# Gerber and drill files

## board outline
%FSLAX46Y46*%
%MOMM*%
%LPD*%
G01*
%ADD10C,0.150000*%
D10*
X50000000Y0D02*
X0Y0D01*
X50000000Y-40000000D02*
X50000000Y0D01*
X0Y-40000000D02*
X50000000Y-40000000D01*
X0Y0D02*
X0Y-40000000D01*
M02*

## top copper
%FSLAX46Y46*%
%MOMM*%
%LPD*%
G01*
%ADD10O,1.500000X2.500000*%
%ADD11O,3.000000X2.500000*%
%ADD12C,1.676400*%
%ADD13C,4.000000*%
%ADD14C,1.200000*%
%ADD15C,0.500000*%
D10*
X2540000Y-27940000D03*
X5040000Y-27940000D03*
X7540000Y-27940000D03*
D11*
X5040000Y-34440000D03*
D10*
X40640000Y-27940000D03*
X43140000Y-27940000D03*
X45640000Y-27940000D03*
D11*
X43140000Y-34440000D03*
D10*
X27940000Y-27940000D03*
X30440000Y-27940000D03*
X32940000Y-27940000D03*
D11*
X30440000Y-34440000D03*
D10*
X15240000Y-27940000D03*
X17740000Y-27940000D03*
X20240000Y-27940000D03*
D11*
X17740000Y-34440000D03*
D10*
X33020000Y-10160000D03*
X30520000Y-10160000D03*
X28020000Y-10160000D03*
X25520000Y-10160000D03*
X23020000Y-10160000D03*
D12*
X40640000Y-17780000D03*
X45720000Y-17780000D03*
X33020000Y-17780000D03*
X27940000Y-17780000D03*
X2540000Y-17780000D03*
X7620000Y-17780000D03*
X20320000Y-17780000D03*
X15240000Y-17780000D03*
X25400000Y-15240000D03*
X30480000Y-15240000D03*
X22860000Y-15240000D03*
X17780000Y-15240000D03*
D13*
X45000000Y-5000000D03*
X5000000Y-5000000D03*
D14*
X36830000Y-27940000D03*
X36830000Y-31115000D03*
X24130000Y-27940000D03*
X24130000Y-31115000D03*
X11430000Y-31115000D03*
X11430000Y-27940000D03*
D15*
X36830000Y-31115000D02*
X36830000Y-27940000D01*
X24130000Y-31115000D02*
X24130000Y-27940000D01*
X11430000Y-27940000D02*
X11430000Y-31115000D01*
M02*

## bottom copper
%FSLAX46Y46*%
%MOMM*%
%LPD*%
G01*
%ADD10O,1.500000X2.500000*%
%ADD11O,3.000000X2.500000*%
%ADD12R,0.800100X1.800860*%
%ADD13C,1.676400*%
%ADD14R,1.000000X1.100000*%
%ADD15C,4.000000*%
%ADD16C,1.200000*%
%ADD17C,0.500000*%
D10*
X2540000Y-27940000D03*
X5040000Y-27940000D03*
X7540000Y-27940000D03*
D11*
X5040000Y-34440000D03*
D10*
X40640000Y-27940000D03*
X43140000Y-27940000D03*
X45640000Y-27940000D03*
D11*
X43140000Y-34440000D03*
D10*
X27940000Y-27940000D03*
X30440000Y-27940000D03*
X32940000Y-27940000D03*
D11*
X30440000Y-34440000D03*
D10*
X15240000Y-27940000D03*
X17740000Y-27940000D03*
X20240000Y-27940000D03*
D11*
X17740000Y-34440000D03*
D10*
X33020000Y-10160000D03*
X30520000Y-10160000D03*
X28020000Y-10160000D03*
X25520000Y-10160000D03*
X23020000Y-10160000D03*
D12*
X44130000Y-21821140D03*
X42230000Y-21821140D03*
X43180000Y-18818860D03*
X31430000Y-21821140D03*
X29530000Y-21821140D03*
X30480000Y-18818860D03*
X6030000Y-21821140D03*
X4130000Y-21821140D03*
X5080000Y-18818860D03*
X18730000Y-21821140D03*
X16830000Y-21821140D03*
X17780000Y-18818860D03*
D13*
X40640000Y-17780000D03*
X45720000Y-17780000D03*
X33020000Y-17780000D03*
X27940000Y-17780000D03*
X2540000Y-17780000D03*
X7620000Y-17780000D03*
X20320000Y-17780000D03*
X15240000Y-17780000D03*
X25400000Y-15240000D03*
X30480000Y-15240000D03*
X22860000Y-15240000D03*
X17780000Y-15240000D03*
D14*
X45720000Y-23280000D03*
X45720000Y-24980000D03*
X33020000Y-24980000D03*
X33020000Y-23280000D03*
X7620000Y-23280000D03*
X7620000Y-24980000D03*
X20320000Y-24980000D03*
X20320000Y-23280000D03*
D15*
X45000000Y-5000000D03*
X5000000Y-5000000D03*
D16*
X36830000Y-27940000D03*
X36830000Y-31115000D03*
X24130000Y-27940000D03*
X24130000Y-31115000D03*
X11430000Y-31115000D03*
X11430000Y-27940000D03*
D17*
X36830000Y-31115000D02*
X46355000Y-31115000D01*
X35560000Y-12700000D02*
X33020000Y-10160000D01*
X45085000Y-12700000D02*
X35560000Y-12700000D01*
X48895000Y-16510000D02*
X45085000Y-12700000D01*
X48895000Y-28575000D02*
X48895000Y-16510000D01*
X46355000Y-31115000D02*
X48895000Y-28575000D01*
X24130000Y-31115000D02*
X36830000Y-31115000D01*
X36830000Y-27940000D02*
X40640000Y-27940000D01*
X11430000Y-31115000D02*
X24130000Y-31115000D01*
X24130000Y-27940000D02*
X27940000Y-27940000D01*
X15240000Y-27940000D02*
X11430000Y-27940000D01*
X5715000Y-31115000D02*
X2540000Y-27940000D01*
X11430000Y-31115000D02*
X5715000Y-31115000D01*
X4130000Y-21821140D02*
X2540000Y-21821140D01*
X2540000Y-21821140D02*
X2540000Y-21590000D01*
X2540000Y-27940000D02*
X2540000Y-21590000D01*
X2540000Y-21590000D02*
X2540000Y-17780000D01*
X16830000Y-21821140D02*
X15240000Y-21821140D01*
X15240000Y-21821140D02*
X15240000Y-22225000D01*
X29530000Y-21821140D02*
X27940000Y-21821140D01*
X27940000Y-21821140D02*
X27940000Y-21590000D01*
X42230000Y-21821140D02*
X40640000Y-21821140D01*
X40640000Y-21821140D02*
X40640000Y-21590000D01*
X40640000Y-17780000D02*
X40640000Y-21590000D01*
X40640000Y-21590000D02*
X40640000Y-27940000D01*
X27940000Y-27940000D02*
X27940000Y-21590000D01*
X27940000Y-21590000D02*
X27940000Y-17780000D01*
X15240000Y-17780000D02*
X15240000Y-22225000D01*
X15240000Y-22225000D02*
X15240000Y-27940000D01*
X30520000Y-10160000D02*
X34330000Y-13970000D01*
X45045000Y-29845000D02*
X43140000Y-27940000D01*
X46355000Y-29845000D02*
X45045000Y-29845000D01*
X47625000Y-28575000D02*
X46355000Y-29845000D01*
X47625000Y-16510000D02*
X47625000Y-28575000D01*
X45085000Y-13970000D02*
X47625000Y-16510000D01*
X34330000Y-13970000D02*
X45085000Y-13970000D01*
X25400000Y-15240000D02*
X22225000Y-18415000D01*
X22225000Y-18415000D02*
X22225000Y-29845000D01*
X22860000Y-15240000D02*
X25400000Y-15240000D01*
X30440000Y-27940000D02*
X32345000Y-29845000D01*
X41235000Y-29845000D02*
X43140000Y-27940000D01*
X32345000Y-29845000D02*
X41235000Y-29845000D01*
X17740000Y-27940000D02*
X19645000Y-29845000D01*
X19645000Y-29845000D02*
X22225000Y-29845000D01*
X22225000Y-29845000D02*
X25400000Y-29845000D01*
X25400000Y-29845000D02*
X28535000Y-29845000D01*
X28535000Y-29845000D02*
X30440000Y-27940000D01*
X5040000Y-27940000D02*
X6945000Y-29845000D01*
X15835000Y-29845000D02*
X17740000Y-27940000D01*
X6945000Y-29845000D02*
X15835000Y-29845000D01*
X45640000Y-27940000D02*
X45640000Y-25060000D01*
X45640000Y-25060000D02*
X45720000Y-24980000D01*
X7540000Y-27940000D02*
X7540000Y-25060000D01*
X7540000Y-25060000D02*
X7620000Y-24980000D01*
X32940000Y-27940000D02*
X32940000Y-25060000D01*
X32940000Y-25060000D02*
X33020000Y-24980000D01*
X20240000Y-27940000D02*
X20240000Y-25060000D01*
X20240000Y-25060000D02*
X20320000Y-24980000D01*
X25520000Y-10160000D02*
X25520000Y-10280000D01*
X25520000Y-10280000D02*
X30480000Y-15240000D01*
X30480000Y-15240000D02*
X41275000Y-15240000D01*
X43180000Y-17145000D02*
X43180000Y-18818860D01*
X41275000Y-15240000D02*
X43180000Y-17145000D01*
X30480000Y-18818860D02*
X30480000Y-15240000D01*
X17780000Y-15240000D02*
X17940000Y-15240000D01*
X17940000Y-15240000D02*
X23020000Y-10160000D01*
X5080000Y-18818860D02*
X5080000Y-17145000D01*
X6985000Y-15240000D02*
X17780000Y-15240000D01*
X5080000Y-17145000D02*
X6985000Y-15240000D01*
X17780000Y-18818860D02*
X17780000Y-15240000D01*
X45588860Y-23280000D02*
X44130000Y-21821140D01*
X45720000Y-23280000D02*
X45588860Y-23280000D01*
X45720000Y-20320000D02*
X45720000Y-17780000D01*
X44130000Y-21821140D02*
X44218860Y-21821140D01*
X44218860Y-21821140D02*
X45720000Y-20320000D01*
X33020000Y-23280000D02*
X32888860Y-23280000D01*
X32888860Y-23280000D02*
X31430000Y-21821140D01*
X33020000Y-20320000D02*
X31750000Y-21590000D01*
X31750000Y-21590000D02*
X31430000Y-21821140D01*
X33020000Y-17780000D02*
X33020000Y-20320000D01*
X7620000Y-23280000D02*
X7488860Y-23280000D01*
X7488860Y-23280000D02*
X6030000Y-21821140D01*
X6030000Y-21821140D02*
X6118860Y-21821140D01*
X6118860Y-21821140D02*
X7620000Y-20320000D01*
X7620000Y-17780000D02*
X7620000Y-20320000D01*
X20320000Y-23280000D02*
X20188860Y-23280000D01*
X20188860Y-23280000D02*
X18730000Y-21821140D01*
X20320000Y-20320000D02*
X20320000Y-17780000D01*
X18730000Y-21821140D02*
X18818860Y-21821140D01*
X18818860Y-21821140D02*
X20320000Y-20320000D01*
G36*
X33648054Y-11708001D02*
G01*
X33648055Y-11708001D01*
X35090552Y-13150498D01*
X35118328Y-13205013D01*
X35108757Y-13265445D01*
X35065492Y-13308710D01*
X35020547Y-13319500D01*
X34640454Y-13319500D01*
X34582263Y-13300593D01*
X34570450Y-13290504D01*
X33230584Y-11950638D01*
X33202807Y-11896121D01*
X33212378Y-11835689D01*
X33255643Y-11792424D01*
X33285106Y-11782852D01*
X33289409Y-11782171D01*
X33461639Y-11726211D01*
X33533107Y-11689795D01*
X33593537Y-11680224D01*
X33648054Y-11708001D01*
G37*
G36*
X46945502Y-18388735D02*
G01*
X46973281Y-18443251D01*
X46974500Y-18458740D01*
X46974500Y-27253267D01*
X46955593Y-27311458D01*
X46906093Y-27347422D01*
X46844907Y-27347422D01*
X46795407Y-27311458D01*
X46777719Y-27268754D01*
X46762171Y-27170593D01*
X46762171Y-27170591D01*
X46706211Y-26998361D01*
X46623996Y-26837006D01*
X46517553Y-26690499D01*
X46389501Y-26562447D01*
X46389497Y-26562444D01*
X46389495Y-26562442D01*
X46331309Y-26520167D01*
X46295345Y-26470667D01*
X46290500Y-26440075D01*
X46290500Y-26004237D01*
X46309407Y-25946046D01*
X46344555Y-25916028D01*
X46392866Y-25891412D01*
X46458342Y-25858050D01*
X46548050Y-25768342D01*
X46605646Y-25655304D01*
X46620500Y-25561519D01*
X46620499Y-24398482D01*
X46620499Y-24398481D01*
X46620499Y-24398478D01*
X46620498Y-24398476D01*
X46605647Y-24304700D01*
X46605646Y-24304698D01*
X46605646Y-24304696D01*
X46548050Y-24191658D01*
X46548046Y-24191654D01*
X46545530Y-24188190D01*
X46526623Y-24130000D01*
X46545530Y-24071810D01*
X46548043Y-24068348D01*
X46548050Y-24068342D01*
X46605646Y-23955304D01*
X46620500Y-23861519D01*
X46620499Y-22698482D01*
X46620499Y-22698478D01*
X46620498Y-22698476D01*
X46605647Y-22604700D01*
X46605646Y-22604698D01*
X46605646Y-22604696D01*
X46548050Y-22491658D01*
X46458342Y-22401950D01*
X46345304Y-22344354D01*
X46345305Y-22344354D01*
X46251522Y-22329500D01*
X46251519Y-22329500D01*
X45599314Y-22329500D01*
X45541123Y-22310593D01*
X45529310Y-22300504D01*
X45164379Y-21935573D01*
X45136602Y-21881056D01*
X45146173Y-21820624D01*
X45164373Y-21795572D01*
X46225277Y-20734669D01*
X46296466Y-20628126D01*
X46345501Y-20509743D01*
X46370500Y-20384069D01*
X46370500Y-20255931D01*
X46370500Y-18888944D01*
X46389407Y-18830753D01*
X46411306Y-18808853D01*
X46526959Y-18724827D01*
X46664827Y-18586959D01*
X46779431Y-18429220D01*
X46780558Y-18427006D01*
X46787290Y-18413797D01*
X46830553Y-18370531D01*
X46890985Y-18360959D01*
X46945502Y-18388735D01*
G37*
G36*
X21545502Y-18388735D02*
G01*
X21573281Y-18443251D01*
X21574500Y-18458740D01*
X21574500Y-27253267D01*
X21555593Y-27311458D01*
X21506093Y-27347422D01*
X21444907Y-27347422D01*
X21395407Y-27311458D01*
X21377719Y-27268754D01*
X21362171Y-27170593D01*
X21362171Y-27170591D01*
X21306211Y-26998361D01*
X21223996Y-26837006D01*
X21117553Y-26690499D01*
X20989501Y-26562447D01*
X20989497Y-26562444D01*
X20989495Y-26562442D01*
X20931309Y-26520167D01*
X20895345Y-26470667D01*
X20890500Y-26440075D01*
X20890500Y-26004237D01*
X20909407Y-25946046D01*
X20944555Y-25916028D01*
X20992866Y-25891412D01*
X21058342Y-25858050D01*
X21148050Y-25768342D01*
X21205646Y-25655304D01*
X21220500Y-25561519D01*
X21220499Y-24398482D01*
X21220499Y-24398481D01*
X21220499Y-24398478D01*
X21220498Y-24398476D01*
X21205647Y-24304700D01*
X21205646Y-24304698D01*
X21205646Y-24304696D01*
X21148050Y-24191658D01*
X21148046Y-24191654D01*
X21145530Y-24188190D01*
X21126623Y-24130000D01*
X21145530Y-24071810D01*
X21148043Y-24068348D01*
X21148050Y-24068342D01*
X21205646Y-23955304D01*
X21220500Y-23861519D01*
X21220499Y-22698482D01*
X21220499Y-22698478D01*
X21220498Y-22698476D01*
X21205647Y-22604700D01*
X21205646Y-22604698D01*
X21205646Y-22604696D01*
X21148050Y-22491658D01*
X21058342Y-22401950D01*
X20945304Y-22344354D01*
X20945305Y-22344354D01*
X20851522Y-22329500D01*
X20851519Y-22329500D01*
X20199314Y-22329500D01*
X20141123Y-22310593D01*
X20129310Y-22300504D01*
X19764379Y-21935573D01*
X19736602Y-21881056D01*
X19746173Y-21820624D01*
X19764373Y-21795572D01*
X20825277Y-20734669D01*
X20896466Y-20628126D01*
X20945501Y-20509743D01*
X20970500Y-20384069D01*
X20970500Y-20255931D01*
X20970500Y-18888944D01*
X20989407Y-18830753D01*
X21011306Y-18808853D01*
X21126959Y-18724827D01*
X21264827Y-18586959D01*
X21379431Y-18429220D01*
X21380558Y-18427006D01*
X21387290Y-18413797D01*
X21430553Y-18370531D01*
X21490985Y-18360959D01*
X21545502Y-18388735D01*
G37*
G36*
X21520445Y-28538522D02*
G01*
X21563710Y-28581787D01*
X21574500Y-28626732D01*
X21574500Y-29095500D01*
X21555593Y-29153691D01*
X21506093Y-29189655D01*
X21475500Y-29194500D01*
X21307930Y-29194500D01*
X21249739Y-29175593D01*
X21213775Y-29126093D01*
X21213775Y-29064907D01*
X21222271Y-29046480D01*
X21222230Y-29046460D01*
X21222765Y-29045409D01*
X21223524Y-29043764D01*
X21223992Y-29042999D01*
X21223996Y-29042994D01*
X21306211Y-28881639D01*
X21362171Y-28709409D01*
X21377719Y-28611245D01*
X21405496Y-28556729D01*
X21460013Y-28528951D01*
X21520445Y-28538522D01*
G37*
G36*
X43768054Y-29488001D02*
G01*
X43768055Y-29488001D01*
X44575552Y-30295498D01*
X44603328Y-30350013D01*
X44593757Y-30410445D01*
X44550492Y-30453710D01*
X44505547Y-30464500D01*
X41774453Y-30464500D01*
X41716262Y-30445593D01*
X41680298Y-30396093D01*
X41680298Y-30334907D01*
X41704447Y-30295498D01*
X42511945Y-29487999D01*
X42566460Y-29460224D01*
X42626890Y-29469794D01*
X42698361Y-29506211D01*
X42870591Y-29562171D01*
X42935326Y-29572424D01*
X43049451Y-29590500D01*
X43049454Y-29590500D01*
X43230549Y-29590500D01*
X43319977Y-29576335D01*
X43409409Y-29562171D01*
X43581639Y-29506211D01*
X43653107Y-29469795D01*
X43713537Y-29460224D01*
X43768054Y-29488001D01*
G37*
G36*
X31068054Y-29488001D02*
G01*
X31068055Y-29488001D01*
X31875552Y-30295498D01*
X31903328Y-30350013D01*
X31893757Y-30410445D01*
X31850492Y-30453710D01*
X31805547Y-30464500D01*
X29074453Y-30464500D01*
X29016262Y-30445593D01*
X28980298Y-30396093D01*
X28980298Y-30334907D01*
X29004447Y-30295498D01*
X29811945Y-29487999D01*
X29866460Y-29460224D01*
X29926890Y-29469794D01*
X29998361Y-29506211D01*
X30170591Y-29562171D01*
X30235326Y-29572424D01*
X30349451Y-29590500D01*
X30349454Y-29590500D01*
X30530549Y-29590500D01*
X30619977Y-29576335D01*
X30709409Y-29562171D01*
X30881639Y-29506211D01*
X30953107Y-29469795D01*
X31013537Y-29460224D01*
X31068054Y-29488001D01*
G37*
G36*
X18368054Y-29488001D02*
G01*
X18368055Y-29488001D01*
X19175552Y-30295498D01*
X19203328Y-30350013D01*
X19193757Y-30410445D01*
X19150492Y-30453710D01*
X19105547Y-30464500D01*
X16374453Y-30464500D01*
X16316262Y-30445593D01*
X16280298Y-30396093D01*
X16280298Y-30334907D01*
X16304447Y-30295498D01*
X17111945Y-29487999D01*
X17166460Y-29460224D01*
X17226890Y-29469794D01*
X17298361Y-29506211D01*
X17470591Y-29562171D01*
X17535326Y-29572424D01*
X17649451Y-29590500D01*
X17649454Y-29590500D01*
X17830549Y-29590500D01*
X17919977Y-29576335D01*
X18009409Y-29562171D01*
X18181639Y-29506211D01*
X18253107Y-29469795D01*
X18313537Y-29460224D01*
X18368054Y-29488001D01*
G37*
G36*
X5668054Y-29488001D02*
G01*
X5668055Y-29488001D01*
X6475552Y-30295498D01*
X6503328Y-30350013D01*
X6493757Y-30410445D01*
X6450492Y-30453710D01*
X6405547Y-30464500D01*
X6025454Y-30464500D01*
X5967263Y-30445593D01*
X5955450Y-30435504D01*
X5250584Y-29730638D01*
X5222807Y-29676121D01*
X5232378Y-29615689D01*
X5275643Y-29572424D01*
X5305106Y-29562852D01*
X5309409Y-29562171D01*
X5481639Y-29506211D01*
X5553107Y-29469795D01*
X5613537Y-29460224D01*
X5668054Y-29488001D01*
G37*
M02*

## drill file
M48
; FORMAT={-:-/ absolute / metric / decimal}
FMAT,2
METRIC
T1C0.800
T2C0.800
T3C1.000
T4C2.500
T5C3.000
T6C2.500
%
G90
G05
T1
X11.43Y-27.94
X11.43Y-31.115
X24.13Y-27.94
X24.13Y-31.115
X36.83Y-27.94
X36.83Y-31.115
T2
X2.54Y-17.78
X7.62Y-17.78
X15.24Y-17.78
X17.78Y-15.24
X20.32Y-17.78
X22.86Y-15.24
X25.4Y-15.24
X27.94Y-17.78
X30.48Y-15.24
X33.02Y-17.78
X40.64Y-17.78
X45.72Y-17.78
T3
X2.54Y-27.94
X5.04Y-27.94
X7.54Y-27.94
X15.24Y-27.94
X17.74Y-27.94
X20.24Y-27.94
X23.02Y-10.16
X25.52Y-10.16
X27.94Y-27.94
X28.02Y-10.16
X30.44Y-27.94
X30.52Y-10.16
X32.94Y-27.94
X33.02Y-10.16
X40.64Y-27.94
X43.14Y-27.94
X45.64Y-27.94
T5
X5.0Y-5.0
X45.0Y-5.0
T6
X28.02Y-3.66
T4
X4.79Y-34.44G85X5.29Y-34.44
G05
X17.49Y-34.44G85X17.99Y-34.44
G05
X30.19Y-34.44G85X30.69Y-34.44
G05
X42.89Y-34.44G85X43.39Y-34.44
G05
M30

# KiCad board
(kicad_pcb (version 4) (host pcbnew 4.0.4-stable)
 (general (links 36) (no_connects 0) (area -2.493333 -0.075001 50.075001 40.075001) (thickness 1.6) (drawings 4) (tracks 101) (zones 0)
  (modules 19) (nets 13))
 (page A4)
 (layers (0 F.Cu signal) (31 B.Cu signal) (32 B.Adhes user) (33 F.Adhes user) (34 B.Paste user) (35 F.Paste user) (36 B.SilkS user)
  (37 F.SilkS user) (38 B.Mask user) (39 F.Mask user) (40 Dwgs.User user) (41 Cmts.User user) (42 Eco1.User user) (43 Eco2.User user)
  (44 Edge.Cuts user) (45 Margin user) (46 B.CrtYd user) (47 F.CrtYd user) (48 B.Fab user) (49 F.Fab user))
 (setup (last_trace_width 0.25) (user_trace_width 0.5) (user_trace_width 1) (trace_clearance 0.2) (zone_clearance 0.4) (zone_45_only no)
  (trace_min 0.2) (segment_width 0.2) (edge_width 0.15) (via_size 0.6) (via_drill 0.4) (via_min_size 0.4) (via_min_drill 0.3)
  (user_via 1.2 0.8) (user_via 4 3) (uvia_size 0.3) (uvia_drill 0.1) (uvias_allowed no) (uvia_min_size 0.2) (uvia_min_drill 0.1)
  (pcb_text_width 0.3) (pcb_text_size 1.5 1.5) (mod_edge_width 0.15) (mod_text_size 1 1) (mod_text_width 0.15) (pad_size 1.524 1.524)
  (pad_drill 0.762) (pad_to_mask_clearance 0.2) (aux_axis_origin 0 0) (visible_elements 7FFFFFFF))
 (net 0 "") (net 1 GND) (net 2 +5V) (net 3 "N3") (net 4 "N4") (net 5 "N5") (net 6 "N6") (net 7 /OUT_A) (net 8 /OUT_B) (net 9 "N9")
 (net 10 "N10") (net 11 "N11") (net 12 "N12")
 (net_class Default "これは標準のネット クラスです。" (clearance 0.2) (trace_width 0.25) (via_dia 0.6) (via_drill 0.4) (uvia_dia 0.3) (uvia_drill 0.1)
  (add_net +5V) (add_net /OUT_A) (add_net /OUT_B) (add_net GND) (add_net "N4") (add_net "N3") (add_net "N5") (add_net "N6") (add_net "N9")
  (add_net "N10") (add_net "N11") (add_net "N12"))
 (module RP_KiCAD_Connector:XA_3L (layer F.Cu) (at 2.54 27.94)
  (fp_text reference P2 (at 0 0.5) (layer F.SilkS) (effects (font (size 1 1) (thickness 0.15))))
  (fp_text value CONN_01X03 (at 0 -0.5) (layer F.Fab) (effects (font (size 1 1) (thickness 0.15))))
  (pad 1 thru_hole oval (at 0 0) (size 1.5 2.5) (drill 1) (layers *.Cu *.Mask F.SilkS) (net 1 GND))
  (pad 2 thru_hole oval (at 2.5 0) (size 1.5 2.5) (drill 1) (layers *.Cu *.Mask F.SilkS) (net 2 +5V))
  (pad 3 thru_hole oval (at 5 0) (size 1.5 2.5) (drill 1) (layers *.Cu *.Mask F.SilkS) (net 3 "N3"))
  (pad "" thru_hole oval (at 2.5 6.5) (size 3 2.5) (drill oval 3 2.5) (layers *.Cu *.Mask F.SilkS)))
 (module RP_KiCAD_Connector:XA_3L (layer F.Cu) (at 40.64 27.94)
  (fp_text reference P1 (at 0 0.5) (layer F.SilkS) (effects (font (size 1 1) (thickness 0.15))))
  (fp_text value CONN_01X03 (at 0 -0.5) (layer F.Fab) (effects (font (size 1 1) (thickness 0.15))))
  (pad 1 thru_hole oval (at 0 0) (size 1.5 2.5) (drill 1) (layers *.Cu *.Mask F.SilkS) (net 1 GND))
  (pad 2 thru_hole oval (at 2.5 0) (size 1.5 2.5) (drill 1) (layers *.Cu *.Mask F.SilkS) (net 2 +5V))
  (pad 3 thru_hole oval (at 5 0) (size 1.5 2.5) (drill 1) (layers *.Cu *.Mask F.SilkS) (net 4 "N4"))
  (pad "" thru_hole oval (at 2.5 6.5) (size 3 2.5) (drill oval 3 2.5) (layers *.Cu *.Mask F.SilkS)))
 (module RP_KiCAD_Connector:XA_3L (layer F.Cu) (at 27.94 27.94)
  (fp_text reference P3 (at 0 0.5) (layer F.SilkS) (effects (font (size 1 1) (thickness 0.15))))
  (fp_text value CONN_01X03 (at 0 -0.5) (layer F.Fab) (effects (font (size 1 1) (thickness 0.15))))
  (pad 1 thru_hole oval (at 0 0) (size 1.5 2.5) (drill 1) (layers *.Cu *.Mask F.SilkS) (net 1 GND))
  (pad 2 thru_hole oval (at 2.5 0) (size 1.5 2.5) (drill 1) (layers *.Cu *.Mask F.SilkS) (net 2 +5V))
  (pad 3 thru_hole oval (at 5 0) (size 1.5 2.5) (drill 1) (layers *.Cu *.Mask F.SilkS) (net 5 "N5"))
  (pad "" thru_hole oval (at 2.5 6.5) (size 3 2.5) (drill oval 3 2.5) (layers *.Cu *.Mask F.SilkS)))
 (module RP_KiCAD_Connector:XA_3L (layer F.Cu) (at 15.24 27.94)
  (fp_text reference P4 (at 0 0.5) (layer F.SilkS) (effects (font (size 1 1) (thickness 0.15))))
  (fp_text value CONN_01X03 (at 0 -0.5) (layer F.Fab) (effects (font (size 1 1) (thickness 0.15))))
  (pad 1 thru_hole oval (at 0 0) (size 1.5 2.5) (drill 1) (layers *.Cu *.Mask F.SilkS) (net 1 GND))
  (pad 2 thru_hole oval (at 2.5 0) (size 1.5 2.5) (drill 1) (layers *.Cu *.Mask F.SilkS) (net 2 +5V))
  (pad 3 thru_hole oval (at 5 0) (size 1.5 2.5) (drill 1) (layers *.Cu *.Mask F.SilkS) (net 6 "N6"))
  (pad "" thru_hole oval (at 2.5 6.5) (size 3 2.5) (drill oval 3 2.5) (layers *.Cu *.Mask F.SilkS)))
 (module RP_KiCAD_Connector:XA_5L (layer F.Cu) (at 33.02 10.16 180)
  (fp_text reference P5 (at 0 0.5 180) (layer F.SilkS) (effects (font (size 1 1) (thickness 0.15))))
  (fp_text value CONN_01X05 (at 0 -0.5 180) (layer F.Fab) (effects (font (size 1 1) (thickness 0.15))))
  (pad 1 thru_hole oval (at 0 0 180) (size 1.5 2.5) (drill 1) (layers *.Cu *.Mask F.SilkS) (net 1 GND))
  (pad 2 thru_hole oval (at 2.5 0 180) (size 1.5 2.5) (drill 1) (layers *.Cu *.Mask F.SilkS) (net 2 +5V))
  (pad 3 thru_hole oval (at 5 0 180) (size 1.5 2.5) (drill 1) (layers *.Cu *.Mask F.SilkS))
  (pad 4 thru_hole oval (at 7.5 0 180) (size 1.5 2.5) (drill 1) (layers *.Cu *.Mask F.SilkS) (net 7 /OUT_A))
  (pad 5 thru_hole oval (at 10 0 180) (size 1.5 2.5) (drill 1) (layers *.Cu *.Mask F.SilkS) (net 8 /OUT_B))
  (pad "" np_thru_hole circle (at 5 6.5 180) (size 2.5 2.5) (drill 2.5) (layers *.Cu *.Mask F.SilkS)))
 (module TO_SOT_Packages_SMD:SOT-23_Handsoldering (layer B.Cu) (at 43.18 20.32 180)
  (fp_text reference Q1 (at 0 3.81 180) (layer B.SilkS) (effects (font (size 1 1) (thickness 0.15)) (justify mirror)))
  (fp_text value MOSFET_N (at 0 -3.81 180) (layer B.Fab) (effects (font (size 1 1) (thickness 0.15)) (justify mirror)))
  (pad G smd rect (at -0.95 -1.50114 180) (size 0.8001 1.80086) (layers B.Cu B.Paste B.Mask) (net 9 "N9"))
  (pad S smd rect (at 0.95 -1.50114 180) (size 0.8001 1.80086) (layers B.Cu B.Paste B.Mask) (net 1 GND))
  (pad D smd rect (at 0 1.50114 180) (size 0.8001 1.80086) (layers B.Cu B.Paste B.Mask) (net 7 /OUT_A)))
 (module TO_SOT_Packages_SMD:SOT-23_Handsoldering (layer B.Cu) (at 30.48 20.32 180)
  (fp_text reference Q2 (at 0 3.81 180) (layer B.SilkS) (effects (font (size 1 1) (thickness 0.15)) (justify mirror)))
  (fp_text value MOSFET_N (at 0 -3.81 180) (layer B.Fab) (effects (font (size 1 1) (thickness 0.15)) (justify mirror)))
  (pad G smd rect (at -0.95 -1.50114 180) (size 0.8001 1.80086) (layers B.Cu B.Paste B.Mask) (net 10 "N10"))
  (pad S smd rect (at 0.95 -1.50114 180) (size 0.8001 1.80086) (layers B.Cu B.Paste B.Mask) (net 1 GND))
  (pad D smd rect (at 0 1.50114 180) (size 0.8001 1.80086) (layers B.Cu B.Paste B.Mask) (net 7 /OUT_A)))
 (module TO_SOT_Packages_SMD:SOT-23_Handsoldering (layer B.Cu) (at 5.08 20.32 180)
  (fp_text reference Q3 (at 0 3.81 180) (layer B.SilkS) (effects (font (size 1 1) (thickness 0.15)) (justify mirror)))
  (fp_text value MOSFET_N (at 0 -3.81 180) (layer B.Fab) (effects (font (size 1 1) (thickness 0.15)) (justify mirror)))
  (pad G smd rect (at -0.95 -1.50114 180) (size 0.8001 1.80086) (layers B.Cu B.Paste B.Mask) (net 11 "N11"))
  (pad S smd rect (at 0.95 -1.50114 180) (size 0.8001 1.80086) (layers B.Cu B.Paste B.Mask) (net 1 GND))
  (pad D smd rect (at 0 1.50114 180) (size 0.8001 1.80086) (layers B.Cu B.Paste B.Mask) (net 8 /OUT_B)))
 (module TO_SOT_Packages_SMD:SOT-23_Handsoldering (layer B.Cu) (at 17.78 20.32 180)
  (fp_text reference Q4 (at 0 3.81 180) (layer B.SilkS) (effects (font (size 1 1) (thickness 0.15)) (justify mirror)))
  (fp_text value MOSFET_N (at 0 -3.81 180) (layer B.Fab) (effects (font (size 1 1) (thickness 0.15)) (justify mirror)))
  (pad G smd rect (at -0.95 -1.50114 180) (size 0.8001 1.80086) (layers B.Cu B.Paste B.Mask) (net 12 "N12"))
  (pad S smd rect (at 0.95 -1.50114 180) (size 0.8001 1.80086) (layers B.Cu B.Paste B.Mask) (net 1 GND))
  (pad D smd rect (at 0 1.50114 180) (size 0.8001 1.80086) (layers B.Cu B.Paste B.Mask) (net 8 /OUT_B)))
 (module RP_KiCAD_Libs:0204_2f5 (layer F.Cu) (at 43.18 17.78)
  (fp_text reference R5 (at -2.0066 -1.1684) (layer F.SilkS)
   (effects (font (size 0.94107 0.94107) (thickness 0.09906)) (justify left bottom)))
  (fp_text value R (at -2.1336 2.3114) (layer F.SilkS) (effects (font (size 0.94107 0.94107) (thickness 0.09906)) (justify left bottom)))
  (pad 1 thru_hole circle (at -2.54 0) (size 1.6764 1.6764) (drill 0.8) (layers *.Cu *.Mask) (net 1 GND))
  (pad 2 thru_hole circle (at 2.54 0) (size 1.6764 1.6764) (drill 0.8) (layers *.Cu *.Mask) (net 9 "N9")))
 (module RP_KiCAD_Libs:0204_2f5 (layer F.Cu) (at 30.48 17.78 180)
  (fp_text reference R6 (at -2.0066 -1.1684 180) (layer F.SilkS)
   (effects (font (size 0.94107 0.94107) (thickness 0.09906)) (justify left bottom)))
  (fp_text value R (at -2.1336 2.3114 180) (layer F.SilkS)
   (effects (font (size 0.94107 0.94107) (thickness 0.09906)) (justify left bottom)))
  (pad 1 thru_hole circle (at -2.54 0 180) (size 1.6764 1.6764) (drill 0.8) (layers *.Cu *.Mask) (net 10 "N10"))
  (pad 2 thru_hole circle (at 2.54 0 180) (size 1.6764 1.6764) (drill 0.8) (layers *.Cu *.Mask) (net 1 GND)))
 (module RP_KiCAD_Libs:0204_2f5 (layer F.Cu) (at 5.08 17.78)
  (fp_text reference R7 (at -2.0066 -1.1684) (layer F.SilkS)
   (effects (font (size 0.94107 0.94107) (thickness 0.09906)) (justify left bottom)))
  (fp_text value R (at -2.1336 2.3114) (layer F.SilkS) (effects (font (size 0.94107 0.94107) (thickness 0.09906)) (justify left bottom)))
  (pad 1 thru_hole circle (at -2.54 0) (size 1.6764 1.6764) (drill 0.8) (layers *.Cu *.Mask) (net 1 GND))
  (pad 2 thru_hole circle (at 2.54 0) (size 1.6764 1.6764) (drill 0.8) (layers *.Cu *.Mask) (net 11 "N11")))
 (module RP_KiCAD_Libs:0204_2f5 (layer F.Cu) (at 17.78 17.78 180)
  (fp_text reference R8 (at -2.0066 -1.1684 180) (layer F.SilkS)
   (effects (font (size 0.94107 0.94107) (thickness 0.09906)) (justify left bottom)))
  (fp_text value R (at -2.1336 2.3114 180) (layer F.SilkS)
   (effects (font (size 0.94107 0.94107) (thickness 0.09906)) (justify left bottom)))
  (pad 1 thru_hole circle (at -2.54 0 180) (size 1.6764 1.6764) (drill 0.8) (layers *.Cu *.Mask) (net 12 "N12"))
  (pad 2 thru_hole circle (at 2.54 0 180) (size 1.6764 1.6764) (drill 0.8) (layers *.Cu *.Mask) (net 1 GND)))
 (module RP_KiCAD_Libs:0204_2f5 (layer F.Cu) (at 27.94 15.24)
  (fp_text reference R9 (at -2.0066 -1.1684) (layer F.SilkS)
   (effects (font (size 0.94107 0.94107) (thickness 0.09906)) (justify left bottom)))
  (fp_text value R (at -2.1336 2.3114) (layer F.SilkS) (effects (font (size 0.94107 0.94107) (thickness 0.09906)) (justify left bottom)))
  (pad 1 thru_hole circle (at -2.54 0) (size 1.6764 1.6764) (drill 0.8) (layers *.Cu *.Mask) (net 2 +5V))
  (pad 2 thru_hole circle (at 2.54 0) (size 1.6764 1.6764) (drill 0.8) (layers *.Cu *.Mask) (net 7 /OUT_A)))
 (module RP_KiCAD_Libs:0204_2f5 (layer F.Cu) (at 20.32 15.24 180)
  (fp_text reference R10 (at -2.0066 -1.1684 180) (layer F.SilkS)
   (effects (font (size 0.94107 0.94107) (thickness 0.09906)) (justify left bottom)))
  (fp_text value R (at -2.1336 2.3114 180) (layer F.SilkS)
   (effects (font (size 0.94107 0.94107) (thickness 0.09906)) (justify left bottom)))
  (pad 1 thru_hole circle (at -2.54 0 180) (size 1.6764 1.6764) (drill 0.8) (layers *.Cu *.Mask) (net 2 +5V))
  (pad 2 thru_hole circle (at 2.54 0 180) (size 1.6764 1.6764) (drill 0.8) (layers *.Cu *.Mask) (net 8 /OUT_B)))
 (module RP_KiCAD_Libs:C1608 (layer B.Cu) (at 45.72 24.13 270)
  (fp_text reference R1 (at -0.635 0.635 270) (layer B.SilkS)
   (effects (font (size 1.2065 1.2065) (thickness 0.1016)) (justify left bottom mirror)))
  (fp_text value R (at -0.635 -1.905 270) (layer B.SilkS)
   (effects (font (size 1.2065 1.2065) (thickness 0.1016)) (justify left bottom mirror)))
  (pad 1 smd rect (at -0.85 0 270) (size 1.1 1) (layers B.Cu B.Paste B.Mask) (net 9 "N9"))
  (pad 2 smd rect (at 0.85 0 270) (size 1.1 1) (layers B.Cu B.Paste B.Mask) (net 4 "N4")))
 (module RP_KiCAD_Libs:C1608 (layer B.Cu) (at 33.02 24.13 90)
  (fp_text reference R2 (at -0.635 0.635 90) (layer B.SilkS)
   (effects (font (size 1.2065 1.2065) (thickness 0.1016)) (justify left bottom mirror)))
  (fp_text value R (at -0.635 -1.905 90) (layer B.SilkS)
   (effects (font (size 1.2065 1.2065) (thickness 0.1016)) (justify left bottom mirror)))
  (pad 1 smd rect (at -0.85 0 90) (size 1.1 1) (layers B.Cu B.Paste B.Mask) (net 5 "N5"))
  (pad 2 smd rect (at 0.85 0 90) (size 1.1 1) (layers B.Cu B.Paste B.Mask) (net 10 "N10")))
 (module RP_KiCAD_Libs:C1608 (layer B.Cu) (at 7.62 24.13 270)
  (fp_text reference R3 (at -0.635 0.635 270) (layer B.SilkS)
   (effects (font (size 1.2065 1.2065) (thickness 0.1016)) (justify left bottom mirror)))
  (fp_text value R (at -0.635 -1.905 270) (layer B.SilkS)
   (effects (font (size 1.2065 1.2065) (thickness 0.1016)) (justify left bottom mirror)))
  (pad 1 smd rect (at -0.85 0 270) (size 1.1 1) (layers B.Cu B.Paste B.Mask) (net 11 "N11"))
  (pad 2 smd rect (at 0.85 0 270) (size 1.1 1) (layers B.Cu B.Paste B.Mask) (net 3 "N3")))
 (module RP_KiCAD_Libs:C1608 (layer B.Cu) (at 20.32 24.13 90)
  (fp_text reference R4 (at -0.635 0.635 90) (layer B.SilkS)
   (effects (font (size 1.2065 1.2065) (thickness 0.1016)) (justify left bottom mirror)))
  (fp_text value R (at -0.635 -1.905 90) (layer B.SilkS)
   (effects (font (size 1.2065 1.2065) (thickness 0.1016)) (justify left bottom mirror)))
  (pad 1 smd rect (at -0.85 0 90) (size 1.1 1) (layers B.Cu B.Paste B.Mask) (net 6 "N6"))
  (pad 2 smd rect (at 0.85 0 90) (size 1.1 1) (layers B.Cu B.Paste B.Mask) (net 12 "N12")))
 (gr_line (start 50 0) (end 0 0) (angle 90) (layer Edge.Cuts) (width 0.15))
 (gr_line (start 50 40) (end 50 0) (angle 90) (layer Edge.Cuts) (width 0.15))
 (gr_line (start 0 40) (end 50 40) (angle 90) (layer Edge.Cuts) (width 0.15))
 (gr_line (start 0 0) (end 0 40) (angle 90) (layer Edge.Cuts) (width 0.15))
 (via (at 45 5) (size 4) (drill 3) (layers F.Cu B.Cu) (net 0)) (via (at 5 5) (size 4) (drill 3) (layers F.Cu B.Cu) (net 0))
 (segment (start 36.83 31.115) (end 46.355 31.115) (width 0.5) (layer B.Cu) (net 1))
 (segment (start 35.56 12.7) (end 33.02 10.16) (width 0.5) (layer B.Cu) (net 1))
 (segment (start 45.085 12.7) (end 35.56 12.7) (width 0.5) (layer B.Cu) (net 1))
 (segment (start 48.895 16.51) (end 45.085 12.7) (width 0.5) (layer B.Cu) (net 1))
 (segment (start 48.895 28.575) (end 48.895 16.51) (width 0.5) (layer B.Cu) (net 1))
 (segment (start 46.355 31.115) (end 48.895 28.575) (width 0.5) (layer B.Cu) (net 1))
 (segment (start 24.13 31.115) (end 36.83 31.115) (width 0.5) (layer B.Cu) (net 1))
 (segment (start 36.83 27.94) (end 40.64 27.94) (width 0.5) (layer B.Cu) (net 1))
 (via (at 36.83 27.94) (size 1.2) (drill 0.8) (layers F.Cu B.Cu) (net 1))
 (segment (start 36.83 31.115) (end 36.83 27.94) (width 0.5) (layer F.Cu) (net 1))
 (via (at 36.83 31.115) (size 1.2) (drill 0.8) (layers F.Cu B.Cu) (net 1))
 (segment (start 11.43 31.115) (end 24.13 31.115) (width 0.5) (layer B.Cu) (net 1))
 (segment (start 24.13 27.94) (end 27.94 27.94) (width 0.5) (layer B.Cu) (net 1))
 (via (at 24.13 27.94) (size 1.2) (drill 0.8) (layers F.Cu B.Cu) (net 1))
 (segment (start 24.13 31.115) (end 24.13 27.94) (width 0.5) (layer F.Cu) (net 1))
 (via (at 24.13 31.115) (size 1.2) (drill 0.8) (layers F.Cu B.Cu) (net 1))
 (segment (start 15.24 27.94) (end 11.43 27.94) (width 0.5) (layer B.Cu) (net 1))
 (segment (start 5.715 31.115) (end 2.54 27.94) (width 0.5) (layer B.Cu) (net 1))
 (segment (start 11.43 31.115) (end 5.715 31.115) (width 0.5) (layer B.Cu) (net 1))
 (via (at 11.43 31.115) (size 1.2) (drill 0.8) (layers F.Cu B.Cu) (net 1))
 (segment (start 11.43 27.94) (end 11.43 31.115) (width 0.5) (layer F.Cu) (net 1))
 (via (at 11.43 27.94) (size 1.2) (drill 0.8) (layers F.Cu B.Cu) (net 1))
 (segment (start 4.13 21.82114) (end 2.54 21.82114) (width 0.5) (layer B.Cu) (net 1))
 (segment (start 2.54 21.82114) (end 2.54 21.59) (width 0.5) (layer B.Cu) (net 1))
 (segment (start 2.54 27.94) (end 2.54 21.59) (width 0.5) (layer B.Cu) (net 1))
 (segment (start 2.54 21.59) (end 2.54 17.78) (width 0.5) (layer B.Cu) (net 1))
 (segment (start 16.83 21.82114) (end 15.24 21.82114) (width 0.5) (layer B.Cu) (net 1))
 (segment (start 15.24 21.82114) (end 15.24 22.225) (width 0.5) (layer B.Cu) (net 1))
 (segment (start 29.53 21.82114) (end 27.94 21.82114) (width 0.5) (layer B.Cu) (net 1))
 (segment (start 27.94 21.82114) (end 27.94 21.59) (width 0.5) (layer B.Cu) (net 1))
 (segment (start 42.23 21.82114) (end 40.64 21.82114) (width 0.5) (layer B.Cu) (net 1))
 (segment (start 40.64 21.82114) (end 40.64 21.59) (width 0.5) (layer B.Cu) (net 1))
 (segment (start 40.64 17.78) (end 40.64 21.59) (width 0.5) (layer B.Cu) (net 1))
 (segment (start 40.64 21.59) (end 40.64 27.94) (width 0.5) (layer B.Cu) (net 1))
 (segment (start 27.94 27.94) (end 27.94 21.59) (width 0.5) (layer B.Cu) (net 1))
 (segment (start 27.94 21.59) (end 27.94 17.78) (width 0.5) (layer B.Cu) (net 1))
 (segment (start 15.24 17.78) (end 15.24 22.225) (width 0.5) (layer B.Cu) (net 1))
 (segment (start 15.24 22.225) (end 15.24 27.94) (width 0.5) (layer B.Cu) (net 1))
 (segment (start 30.52 10.16) (end 34.33 13.97) (width 0.5) (layer B.Cu) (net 2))
 (segment (start 45.045 29.845) (end 43.14 27.94) (width 0.5) (layer B.Cu) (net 2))
 (segment (start 46.355 29.845) (end 45.045 29.845) (width 0.5) (layer B.Cu) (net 2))
 (segment (start 47.625 28.575) (end 46.355 29.845) (width 0.5) (layer B.Cu) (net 2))
 (segment (start 47.625 16.51) (end 47.625 28.575) (width 0.5) (layer B.Cu) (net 2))
 (segment (start 45.085 13.97) (end 47.625 16.51) (width 0.5) (layer B.Cu) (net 2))
 (segment (start 34.33 13.97) (end 45.085 13.97) (width 0.5) (layer B.Cu) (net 2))
 (segment (start 25.4 15.24) (end 22.225 18.415) (width 0.5) (layer B.Cu) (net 2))
 (segment (start 22.225 18.415) (end 22.225 29.845) (width 0.5) (layer B.Cu) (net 2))
 (segment (start 22.86 15.24) (end 25.4 15.24) (width 0.5) (layer B.Cu) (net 2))
 (segment (start 30.44 27.94) (end 32.345 29.845) (width 0.5) (layer B.Cu) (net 2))
 (segment (start 41.235 29.845) (end 43.14 27.94) (width 0.5) (layer B.Cu) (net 2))
 (segment (start 32.345 29.845) (end 41.235 29.845) (width 0.5) (layer B.Cu) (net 2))
 (segment (start 17.74 27.94) (end 19.645 29.845) (width 0.5) (layer B.Cu) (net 2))
 (segment (start 19.645 29.845) (end 22.225 29.845) (width 0.5) (layer B.Cu) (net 2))
 (segment (start 22.225 29.845) (end 25.4 29.845) (width 0.5) (layer B.Cu) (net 2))
 (segment (start 25.4 29.845) (end 28.535 29.845) (width 0.5) (layer B.Cu) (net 2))
 (segment (start 28.535 29.845) (end 30.44 27.94) (width 0.5) (layer B.Cu) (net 2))
 (segment (start 5.04 27.94) (end 6.945 29.845) (width 0.5) (layer B.Cu) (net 2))
 (segment (start 15.835 29.845) (end 17.74 27.94) (width 0.5) (layer B.Cu) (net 2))
 (segment (start 6.945 29.845) (end 15.835 29.845) (width 0.5) (layer B.Cu) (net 2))
 (segment (start 45.64 27.94) (end 45.64 25.06) (width 0.5) (layer B.Cu) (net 4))
 (segment (start 45.64 25.06) (end 45.72 24.98) (width 0.5) (layer B.Cu) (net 4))
 (segment (start 7.54 27.94) (end 7.54 25.06) (width 0.5) (layer B.Cu) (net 3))
 (segment (start 7.54 25.06) (end 7.62 24.98) (width 0.5) (layer B.Cu) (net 3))
 (segment (start 32.94 27.94) (end 32.94 25.06) (width 0.5) (layer B.Cu) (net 5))
 (segment (start 32.94 25.06) (end 33.02 24.98) (width 0.5) (layer B.Cu) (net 5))
 (segment (start 20.24 27.94) (end 20.24 25.06) (width 0.5) (layer B.Cu) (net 6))
 (segment (start 20.24 25.06) (end 20.32 24.98) (width 0.5) (layer B.Cu) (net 6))
 (segment (start 25.52 10.16) (end 25.52 10.28) (width 0.5) (layer B.Cu) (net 7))
 (segment (start 25.52 10.28) (end 30.48 15.24) (width 0.5) (layer B.Cu) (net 7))
 (segment (start 30.48 15.24) (end 41.275 15.24) (width 0.5) (layer B.Cu) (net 7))
 (segment (start 43.18 17.145) (end 43.18 18.81886) (width 0.5) (layer B.Cu) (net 7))
 (segment (start 41.275 15.24) (end 43.18 17.145) (width 0.5) (layer B.Cu) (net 7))
 (segment (start 30.48 18.81886) (end 30.48 15.24) (width 0.5) (layer B.Cu) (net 7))
 (segment (start 17.78 15.24) (end 17.94 15.24) (width 0.5) (layer B.Cu) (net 8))
 (segment (start 17.94 15.24) (end 23.02 10.16) (width 0.5) (layer B.Cu) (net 8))
 (segment (start 5.08 18.81886) (end 5.08 17.145) (width 0.5) (layer B.Cu) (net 8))
 (segment (start 6.985 15.24) (end 17.78 15.24) (width 0.5) (layer B.Cu) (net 8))
 (segment (start 5.08 17.145) (end 6.985 15.24) (width 0.5) (layer B.Cu) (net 8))
 (segment (start 17.78 18.81886) (end 17.78 15.24) (width 0.5) (layer B.Cu) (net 8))
 (segment (start 45.58886 23.28) (end 44.13 21.82114) (width 0.5) (layer B.Cu) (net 9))
 (segment (start 45.72 23.28) (end 45.58886 23.28) (width 0.5) (layer B.Cu) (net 9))
 (segment (start 45.72 20.32) (end 45.72 17.78) (width 0.5) (layer B.Cu) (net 9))
 (segment (start 44.13 21.82114) (end 44.21886 21.82114) (width 0.5) (layer B.Cu) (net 9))
 (segment (start 44.21886 21.82114) (end 45.72 20.32) (width 0.5) (layer B.Cu) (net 9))
 (segment (start 33.02 23.28) (end 32.88886 23.28) (width 0.5) (layer B.Cu) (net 10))
 (segment (start 32.88886 23.28) (end 31.43 21.82114) (width 0.5) (layer B.Cu) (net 10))
 (segment (start 33.02 20.32) (end 31.75 21.59) (width 0.5) (layer B.Cu) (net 10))
 (segment (start 31.75 21.59) (end 31.43 21.82114) (width 0.5) (layer B.Cu) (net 10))
 (segment (start 33.02 17.78) (end 33.02 20.32) (width 0.5) (layer B.Cu) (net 10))
 (segment (start 7.62 23.28) (end 7.48886 23.28) (width 0.5) (layer B.Cu) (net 11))
 (segment (start 7.48886 23.28) (end 6.03 21.82114) (width 0.5) (layer B.Cu) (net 11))
 (segment (start 6.03 21.82114) (end 6.11886 21.82114) (width 0.5) (layer B.Cu) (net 11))
 (segment (start 6.11886 21.82114) (end 7.62 20.32) (width 0.5) (layer B.Cu) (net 11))
 (segment (start 7.62 17.78) (end 7.62 20.32) (width 0.5) (layer B.Cu) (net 11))
 (segment (start 20.32 23.28) (end 20.18886 23.28) (width 0.5) (layer B.Cu) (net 12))
 (segment (start 20.18886 23.28) (end 18.73 21.82114) (width 0.5) (layer B.Cu) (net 12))
 (segment (start 20.32 20.32) (end 20.32 17.78) (width 0.5) (layer B.Cu) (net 12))
 (segment (start 18.73 21.82114) (end 18.81886 21.82114) (width 0.5) (layer B.Cu) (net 12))
 (segment (start 18.81886 21.82114) (end 20.32 20.32) (width 0.5) (layer B.Cu) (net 12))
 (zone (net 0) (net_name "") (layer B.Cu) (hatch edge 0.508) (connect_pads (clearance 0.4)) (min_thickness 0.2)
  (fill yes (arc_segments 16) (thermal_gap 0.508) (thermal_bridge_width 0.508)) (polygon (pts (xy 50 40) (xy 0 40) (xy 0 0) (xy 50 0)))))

